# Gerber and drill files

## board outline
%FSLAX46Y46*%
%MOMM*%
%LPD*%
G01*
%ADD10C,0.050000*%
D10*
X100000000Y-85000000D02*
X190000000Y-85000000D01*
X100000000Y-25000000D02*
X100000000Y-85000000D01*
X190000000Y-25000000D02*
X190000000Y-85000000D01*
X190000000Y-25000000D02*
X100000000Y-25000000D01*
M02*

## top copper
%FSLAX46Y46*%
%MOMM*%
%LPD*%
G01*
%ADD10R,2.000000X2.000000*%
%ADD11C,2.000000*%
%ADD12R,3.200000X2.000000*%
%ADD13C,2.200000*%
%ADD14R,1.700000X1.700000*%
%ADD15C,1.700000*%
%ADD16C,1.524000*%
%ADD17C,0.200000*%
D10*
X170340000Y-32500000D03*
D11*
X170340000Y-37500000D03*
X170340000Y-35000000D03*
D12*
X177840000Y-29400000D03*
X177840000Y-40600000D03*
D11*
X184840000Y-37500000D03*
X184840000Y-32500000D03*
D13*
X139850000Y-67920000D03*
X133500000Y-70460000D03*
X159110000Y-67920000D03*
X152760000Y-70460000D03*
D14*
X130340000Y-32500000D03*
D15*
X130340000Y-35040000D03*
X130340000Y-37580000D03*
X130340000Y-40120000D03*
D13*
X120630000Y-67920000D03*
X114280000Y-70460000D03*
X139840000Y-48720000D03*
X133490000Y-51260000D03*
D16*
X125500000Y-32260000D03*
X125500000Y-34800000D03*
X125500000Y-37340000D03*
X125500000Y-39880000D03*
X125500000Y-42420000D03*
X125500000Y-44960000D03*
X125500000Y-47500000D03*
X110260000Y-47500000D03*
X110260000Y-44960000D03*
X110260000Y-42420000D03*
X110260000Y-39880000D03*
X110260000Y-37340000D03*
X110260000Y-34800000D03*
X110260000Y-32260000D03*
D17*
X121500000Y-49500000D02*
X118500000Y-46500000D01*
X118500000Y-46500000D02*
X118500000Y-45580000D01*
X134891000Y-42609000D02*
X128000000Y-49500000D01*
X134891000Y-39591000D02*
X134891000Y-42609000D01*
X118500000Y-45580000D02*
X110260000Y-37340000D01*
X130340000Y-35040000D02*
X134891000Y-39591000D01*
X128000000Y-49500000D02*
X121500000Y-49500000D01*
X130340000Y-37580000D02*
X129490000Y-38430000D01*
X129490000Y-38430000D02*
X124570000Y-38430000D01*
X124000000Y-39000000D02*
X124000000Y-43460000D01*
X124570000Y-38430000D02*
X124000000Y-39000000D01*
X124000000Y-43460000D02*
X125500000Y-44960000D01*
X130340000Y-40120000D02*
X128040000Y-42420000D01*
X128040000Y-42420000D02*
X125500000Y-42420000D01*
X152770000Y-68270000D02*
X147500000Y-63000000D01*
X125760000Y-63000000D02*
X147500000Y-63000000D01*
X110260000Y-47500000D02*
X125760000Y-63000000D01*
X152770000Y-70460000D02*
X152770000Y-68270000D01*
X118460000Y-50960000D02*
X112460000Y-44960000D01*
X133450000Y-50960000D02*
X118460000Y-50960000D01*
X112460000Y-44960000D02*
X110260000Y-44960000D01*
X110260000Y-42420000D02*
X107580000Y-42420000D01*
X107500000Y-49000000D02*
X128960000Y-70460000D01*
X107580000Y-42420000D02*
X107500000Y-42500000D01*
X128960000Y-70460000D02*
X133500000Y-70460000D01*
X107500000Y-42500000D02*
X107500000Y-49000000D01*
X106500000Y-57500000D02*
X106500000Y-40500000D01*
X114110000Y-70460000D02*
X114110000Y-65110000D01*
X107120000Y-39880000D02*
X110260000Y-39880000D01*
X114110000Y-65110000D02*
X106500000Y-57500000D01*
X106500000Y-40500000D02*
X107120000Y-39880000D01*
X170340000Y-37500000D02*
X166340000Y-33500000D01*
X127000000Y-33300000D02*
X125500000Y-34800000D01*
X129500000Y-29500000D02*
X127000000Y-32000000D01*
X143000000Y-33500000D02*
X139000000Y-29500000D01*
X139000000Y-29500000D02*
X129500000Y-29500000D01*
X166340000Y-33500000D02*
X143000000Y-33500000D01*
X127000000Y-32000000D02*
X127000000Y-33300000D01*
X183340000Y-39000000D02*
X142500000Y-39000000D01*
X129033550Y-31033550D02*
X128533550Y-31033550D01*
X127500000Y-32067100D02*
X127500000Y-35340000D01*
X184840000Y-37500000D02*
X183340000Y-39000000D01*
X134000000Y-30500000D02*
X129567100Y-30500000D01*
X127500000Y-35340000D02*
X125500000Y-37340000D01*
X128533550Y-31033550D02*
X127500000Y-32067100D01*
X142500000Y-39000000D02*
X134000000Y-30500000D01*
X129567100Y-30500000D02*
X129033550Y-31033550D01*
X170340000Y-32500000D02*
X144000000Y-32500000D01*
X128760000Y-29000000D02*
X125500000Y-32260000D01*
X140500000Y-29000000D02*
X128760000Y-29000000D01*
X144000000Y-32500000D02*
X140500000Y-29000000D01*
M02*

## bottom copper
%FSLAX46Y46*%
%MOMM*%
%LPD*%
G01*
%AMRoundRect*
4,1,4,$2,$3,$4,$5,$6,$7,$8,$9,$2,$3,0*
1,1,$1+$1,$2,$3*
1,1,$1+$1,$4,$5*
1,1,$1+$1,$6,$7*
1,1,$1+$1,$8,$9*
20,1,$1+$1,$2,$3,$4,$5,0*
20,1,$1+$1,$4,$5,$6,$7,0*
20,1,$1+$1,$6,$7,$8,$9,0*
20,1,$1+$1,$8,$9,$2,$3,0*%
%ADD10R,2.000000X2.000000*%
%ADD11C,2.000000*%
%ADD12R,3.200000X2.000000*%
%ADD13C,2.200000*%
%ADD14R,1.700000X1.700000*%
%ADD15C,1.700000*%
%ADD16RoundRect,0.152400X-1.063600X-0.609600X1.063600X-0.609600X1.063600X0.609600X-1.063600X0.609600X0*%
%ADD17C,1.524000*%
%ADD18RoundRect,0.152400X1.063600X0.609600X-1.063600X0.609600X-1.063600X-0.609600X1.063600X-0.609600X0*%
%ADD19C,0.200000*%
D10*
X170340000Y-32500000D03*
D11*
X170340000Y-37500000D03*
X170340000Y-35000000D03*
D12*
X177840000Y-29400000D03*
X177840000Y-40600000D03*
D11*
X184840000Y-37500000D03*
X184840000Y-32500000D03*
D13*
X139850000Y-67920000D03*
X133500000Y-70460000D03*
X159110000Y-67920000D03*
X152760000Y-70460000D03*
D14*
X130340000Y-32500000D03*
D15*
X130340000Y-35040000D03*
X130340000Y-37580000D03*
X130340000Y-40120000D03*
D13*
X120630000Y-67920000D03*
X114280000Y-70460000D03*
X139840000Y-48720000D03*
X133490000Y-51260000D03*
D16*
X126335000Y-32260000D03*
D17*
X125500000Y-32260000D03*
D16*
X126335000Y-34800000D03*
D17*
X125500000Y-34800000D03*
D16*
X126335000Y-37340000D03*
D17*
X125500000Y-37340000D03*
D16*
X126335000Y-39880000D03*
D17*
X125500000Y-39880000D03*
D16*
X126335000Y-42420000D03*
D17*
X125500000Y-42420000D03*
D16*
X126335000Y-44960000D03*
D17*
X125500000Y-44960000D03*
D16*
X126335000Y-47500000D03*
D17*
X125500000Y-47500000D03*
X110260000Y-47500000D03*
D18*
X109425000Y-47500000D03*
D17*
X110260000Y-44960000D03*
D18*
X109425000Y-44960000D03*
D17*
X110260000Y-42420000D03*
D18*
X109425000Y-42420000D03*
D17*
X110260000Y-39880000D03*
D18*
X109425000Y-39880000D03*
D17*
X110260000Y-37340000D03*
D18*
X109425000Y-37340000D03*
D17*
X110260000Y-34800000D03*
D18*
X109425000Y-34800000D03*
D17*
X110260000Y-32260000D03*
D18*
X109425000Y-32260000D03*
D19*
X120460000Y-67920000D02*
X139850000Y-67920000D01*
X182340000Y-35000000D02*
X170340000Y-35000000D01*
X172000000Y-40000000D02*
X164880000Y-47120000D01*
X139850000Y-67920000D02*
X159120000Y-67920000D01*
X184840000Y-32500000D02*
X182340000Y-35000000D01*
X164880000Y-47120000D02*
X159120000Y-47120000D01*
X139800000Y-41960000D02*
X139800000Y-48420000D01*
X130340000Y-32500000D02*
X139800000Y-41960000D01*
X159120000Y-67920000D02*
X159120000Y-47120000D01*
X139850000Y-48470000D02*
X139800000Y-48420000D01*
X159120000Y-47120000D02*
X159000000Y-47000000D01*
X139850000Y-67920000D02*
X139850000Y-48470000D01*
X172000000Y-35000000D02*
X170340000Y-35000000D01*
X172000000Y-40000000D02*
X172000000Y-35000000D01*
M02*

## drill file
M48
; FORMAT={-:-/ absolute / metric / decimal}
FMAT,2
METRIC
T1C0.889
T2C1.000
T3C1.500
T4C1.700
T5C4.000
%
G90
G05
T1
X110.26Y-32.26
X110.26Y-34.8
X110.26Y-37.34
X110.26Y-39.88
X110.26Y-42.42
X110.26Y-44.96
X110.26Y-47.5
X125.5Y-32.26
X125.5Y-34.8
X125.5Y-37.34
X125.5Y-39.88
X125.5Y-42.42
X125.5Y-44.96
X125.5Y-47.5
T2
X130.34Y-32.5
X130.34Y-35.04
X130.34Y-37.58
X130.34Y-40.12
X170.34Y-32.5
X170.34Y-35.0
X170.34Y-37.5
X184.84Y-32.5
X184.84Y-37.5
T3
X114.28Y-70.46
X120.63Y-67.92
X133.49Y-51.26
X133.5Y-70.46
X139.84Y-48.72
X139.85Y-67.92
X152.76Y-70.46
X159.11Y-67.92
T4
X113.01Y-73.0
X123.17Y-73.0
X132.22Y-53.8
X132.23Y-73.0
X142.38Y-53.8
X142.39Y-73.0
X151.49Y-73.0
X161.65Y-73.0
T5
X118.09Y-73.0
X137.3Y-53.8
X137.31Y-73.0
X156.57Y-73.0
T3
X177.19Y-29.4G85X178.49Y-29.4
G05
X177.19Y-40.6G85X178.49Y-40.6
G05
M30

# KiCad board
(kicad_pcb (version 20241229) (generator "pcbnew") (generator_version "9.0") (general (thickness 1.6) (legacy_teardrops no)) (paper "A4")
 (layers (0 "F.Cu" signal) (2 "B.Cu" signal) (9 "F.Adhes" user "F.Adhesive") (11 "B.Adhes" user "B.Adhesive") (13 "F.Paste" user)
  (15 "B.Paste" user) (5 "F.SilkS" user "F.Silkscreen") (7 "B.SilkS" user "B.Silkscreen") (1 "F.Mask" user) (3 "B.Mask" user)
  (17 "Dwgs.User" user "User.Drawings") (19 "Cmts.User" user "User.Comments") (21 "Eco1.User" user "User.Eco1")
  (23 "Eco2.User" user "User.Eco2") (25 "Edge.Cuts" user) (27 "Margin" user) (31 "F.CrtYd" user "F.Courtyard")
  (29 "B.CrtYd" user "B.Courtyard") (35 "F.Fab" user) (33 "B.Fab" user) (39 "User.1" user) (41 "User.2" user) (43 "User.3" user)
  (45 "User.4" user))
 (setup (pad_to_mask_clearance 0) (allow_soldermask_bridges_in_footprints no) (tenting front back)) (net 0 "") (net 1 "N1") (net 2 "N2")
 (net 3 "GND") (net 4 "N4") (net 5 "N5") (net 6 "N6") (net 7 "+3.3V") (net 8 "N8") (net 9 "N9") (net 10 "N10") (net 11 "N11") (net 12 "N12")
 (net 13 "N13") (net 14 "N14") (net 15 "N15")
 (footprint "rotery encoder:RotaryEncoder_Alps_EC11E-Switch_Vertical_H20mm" (layer "F.Cu") (at 170.34 32.5)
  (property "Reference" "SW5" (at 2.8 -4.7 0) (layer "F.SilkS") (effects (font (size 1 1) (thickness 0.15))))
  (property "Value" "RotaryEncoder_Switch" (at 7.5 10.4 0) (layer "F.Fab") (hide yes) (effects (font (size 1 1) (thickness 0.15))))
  (pad "A" thru_hole rect (at 0 0) (size 2 2) (drill 1) (layers "*.Cu" "*.Mask") (remove_unused_layers no) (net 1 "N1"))
  (pad "B" thru_hole circle (at 0 5) (size 2 2) (drill 1) (layers "*.Cu" "*.Mask") (remove_unused_layers no) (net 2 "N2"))
  (pad "C" thru_hole circle (at 0 2.5) (size 2 2) (drill 1) (layers "*.Cu" "*.Mask") (remove_unused_layers no) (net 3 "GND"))
  (pad "MP" thru_hole rect (at 7.5 -3.1) (size 3.2 2) (drill oval 2.8 1.5) (layers "*.Cu" "*.Mask") (remove_unused_layers no))
  (pad "MP" thru_hole rect (at 7.5 8.1) (size 3.2 2) (drill oval 2.8 1.5) (layers "*.Cu" "*.Mask") (remove_unused_layers no))
  (pad "S1" thru_hole circle (at 14.5 5) (size 2 2) (drill 1) (layers "*.Cu" "*.Mask") (remove_unused_layers no) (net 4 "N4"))
  (pad "S2" thru_hole circle (at 14.5 0) (size 2 2) (drill 1) (layers "*.Cu" "*.Mask") (remove_unused_layers no) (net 3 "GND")))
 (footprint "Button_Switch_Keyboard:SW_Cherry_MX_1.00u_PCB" (layer "F.Cu") (at 139.85 67.92)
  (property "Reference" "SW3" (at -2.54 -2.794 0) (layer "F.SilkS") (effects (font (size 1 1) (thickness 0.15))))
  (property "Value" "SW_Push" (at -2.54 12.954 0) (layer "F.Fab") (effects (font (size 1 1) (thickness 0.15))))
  (pad "" np_thru_hole circle (at -7.62 5.08) (size 1.7 1.7) (drill 1.7) (layers "*.Cu" "*.Mask"))
  (pad "" np_thru_hole circle (at -2.54 5.08) (size 4 4) (drill 4) (layers "*.Cu" "*.Mask"))
  (pad "" np_thru_hole circle (at 2.54 5.08) (size 1.7 1.7) (drill 1.7) (layers "*.Cu" "*.Mask"))
  (pad "1" thru_hole circle (at 0 0) (size 2.2 2.2) (drill 1.5) (layers "*.Cu" "*.Mask") (remove_unused_layers no) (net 3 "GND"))
  (pad "2" thru_hole circle (at -6.35 2.54) (size 2.2 2.2) (drill 1.5) (layers "*.Cu" "*.Mask") (remove_unused_layers no) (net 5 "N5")))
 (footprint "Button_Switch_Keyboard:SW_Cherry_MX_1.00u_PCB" (layer "F.Cu") (at 159.11 67.92)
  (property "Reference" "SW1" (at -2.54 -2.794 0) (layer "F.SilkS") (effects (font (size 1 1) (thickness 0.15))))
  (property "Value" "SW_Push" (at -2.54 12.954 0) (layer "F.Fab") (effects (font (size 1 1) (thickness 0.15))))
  (pad "" np_thru_hole circle (at -7.62 5.08) (size 1.7 1.7) (drill 1.7) (layers "*.Cu" "*.Mask"))
  (pad "" np_thru_hole circle (at -2.54 5.08) (size 4 4) (drill 4) (layers "*.Cu" "*.Mask"))
  (pad "" np_thru_hole circle (at 2.54 5.08) (size 1.7 1.7) (drill 1.7) (layers "*.Cu" "*.Mask"))
  (pad "1" thru_hole circle (at 0 0) (size 2.2 2.2) (drill 1.5) (layers "*.Cu" "*.Mask") (remove_unused_layers no) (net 3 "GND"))
  (pad "2" thru_hole circle (at -6.35 2.54) (size 2.2 2.2) (drill 1.5) (layers "*.Cu" "*.Mask") (remove_unused_layers no) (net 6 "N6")))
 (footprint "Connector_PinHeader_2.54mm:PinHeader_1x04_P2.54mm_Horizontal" (layer "F.Cu") (at 130.34 32.5)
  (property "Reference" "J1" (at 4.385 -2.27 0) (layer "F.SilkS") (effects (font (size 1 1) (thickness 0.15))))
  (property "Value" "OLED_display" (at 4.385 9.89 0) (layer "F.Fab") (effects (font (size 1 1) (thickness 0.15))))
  (pad "1" thru_hole rect (at 0 0) (size 1.7 1.7) (drill 1) (layers "*.Cu" "*.Mask") (remove_unused_layers no) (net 3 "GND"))
  (pad "2" thru_hole circle (at 0 2.54) (size 1.7 1.7) (drill 1) (layers "*.Cu" "*.Mask") (remove_unused_layers no) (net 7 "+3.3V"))
  (pad "3" thru_hole circle (at 0 5.08) (size 1.7 1.7) (drill 1) (layers "*.Cu" "*.Mask") (remove_unused_layers no) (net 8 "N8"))
  (pad "4" thru_hole circle (at 0 7.62) (size 1.7 1.7) (drill 1) (layers "*.Cu" "*.Mask") (remove_unused_layers no) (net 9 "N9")))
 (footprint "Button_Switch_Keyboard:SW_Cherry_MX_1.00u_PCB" (layer "F.Cu") (at 120.63 67.92)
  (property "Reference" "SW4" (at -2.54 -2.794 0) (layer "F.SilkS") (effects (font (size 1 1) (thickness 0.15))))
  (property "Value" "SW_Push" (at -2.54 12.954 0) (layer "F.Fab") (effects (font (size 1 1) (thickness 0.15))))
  (pad "" np_thru_hole circle (at -7.62 5.08) (size 1.7 1.7) (drill 1.7) (layers "*.Cu" "*.Mask"))
  (pad "" np_thru_hole circle (at -2.54 5.08) (size 4 4) (drill 4) (layers "*.Cu" "*.Mask"))
  (pad "" np_thru_hole circle (at 2.54 5.08) (size 1.7 1.7) (drill 1.7) (layers "*.Cu" "*.Mask"))
  (pad "1" thru_hole circle (at 0 0) (size 2.2 2.2) (drill 1.5) (layers "*.Cu" "*.Mask") (remove_unused_layers no) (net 3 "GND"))
  (pad "2" thru_hole circle (at -6.35 2.54) (size 2.2 2.2) (drill 1.5) (layers "*.Cu" "*.Mask") (remove_unused_layers no) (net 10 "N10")))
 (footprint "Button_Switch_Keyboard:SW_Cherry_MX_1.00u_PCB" (layer "F.Cu") (at 139.84 48.72)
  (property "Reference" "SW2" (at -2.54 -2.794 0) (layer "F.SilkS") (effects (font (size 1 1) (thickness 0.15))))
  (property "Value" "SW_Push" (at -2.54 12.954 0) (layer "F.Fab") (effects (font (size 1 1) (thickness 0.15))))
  (pad "" np_thru_hole circle (at -7.62 5.08) (size 1.7 1.7) (drill 1.7) (layers "*.Cu" "*.Mask"))
  (pad "" np_thru_hole circle (at -2.54 5.08) (size 4 4) (drill 4) (layers "*.Cu" "*.Mask"))
  (pad "" np_thru_hole circle (at 2.54 5.08) (size 1.7 1.7) (drill 1.7) (layers "*.Cu" "*.Mask"))
  (pad "1" thru_hole circle (at 0 0) (size 2.2 2.2) (drill 1.5) (layers "*.Cu" "*.Mask") (remove_unused_layers no) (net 3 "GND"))
  (pad "2" thru_hole circle (at -6.35 2.54) (size 2.2 2.2) (drill 1.5) (layers "*.Cu" "*.Mask") (remove_unused_layers no) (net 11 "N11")))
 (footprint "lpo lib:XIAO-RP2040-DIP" (layer "B.Cu") (at 117.88 39.88 180)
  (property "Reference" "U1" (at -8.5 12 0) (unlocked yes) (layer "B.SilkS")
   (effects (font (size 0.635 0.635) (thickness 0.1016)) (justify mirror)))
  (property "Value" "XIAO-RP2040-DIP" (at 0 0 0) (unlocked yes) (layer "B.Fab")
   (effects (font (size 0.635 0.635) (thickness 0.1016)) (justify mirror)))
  (pad "1" smd roundrect (at -8.455 7.62) (size 2.432 1.524) (layers "B.Cu" "B.Mask") (roundrect_rratio 0.1) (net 1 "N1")
   (thermal_bridge_angle 45))
  (pad "1" thru_hole circle (at -7.62 7.62) (size 1.524 1.524) (drill 0.889) (layers "*.Cu" "*.Mask") (remove_unused_layers no) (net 1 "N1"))
  (pad "2" smd roundrect (at -8.455 5.08) (size 2.432 1.524) (layers "B.Cu" "B.Mask") (roundrect_rratio 0.1) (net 2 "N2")
   (thermal_bridge_angle 45))
  (pad "2" thru_hole circle (at -7.62 5.08) (size 1.524 1.524) (drill 0.889) (layers "*.Cu" "*.Mask") (remove_unused_layers no) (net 2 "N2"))
  (pad "3" smd roundrect (at -8.455 2.54) (size 2.432 1.524) (layers "B.Cu" "B.Mask") (roundrect_rratio 0.1) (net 4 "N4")
   (thermal_bridge_angle 45))
  (pad "3" thru_hole circle (at -7.62 2.54) (size 1.524 1.524) (drill 0.889) (layers "*.Cu" "*.Mask") (remove_unused_layers no) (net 4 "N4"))
  (pad "4" smd roundrect (at -8.455 0) (size 2.432 1.524) (layers "B.Cu" "B.Mask") (roundrect_rratio 0.1) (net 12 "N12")
   (thermal_bridge_angle 45))
  (pad "4" thru_hole circle (at -7.62 0) (size 1.524 1.524) (drill 0.889) (layers "*.Cu" "*.Mask") (remove_unused_layers no) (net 12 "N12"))
  (pad "5" smd roundrect (at -8.455 -2.54) (size 2.432 1.524) (layers "B.Cu" "B.Mask") (roundrect_rratio 0.1) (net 9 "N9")
   (thermal_bridge_angle 45))
  (pad "5" thru_hole circle (at -7.62 -2.54) (size 1.524 1.524) (drill 0.889) (layers "*.Cu" "*.Mask") (remove_unused_layers no)
   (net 9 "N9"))
  (pad "6" smd roundrect (at -8.455 -5.08) (size 2.432 1.524) (layers "B.Cu" "B.Mask") (roundrect_rratio 0.1) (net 8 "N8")
   (thermal_bridge_angle 45))
  (pad "6" thru_hole circle (at -7.62 -5.08) (size 1.524 1.524) (drill 0.889) (layers "*.Cu" "*.Mask") (remove_unused_layers no)
   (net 8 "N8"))
  (pad "7" smd roundrect (at -8.455 -7.62) (size 2.432 1.524) (layers "B.Cu" "B.Mask") (roundrect_rratio 0.1) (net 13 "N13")
   (thermal_bridge_angle 45))
  (pad "7" thru_hole circle (at -7.62 -7.62) (size 1.524 1.524) (drill 0.889) (layers "*.Cu" "*.Mask") (remove_unused_layers no)
   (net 13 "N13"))
  (pad "8" thru_hole circle (at 7.62 -7.62 180) (size 1.524 1.524) (drill 0.889) (layers "*.Cu" "*.Mask") (remove_unused_layers no)
   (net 6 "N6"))
  (pad "8" smd roundrect (at 8.455 -7.62 180) (size 2.432 1.524) (layers "B.Cu" "B.Mask") (roundrect_rratio 0.1) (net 6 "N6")
   (thermal_bridge_angle 45))
  (pad "9" thru_hole circle (at 7.62 -5.08 180) (size 1.524 1.524) (drill 0.889) (layers "*.Cu" "*.Mask") (remove_unused_layers no)
   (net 11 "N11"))
  (pad "9" smd roundrect (at 8.455 -5.08 180) (size 2.432 1.524) (layers "B.Cu" "B.Mask") (roundrect_rratio 0.1) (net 11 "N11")
   (thermal_bridge_angle 45))
  (pad "10" thru_hole circle (at 7.62 -2.54 180) (size 1.524 1.524) (drill 0.889) (layers "*.Cu" "*.Mask") (remove_unused_layers no)
   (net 5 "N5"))
  (pad "10" smd roundrect (at 8.455 -2.54 180) (size 2.432 1.524) (layers "B.Cu" "B.Mask") (roundrect_rratio 0.1) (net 5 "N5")
   (thermal_bridge_angle 45))
  (pad "11" thru_hole circle (at 7.62 0 180) (size 1.524 1.524) (drill 0.889) (layers "*.Cu" "*.Mask") (remove_unused_layers no)
   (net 10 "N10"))
  (pad "11" smd roundrect (at 8.455 0 180) (size 2.432 1.524) (layers "B.Cu" "B.Mask") (roundrect_rratio 0.1) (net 10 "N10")
   (thermal_bridge_angle 45))
  (pad "12" thru_hole circle (at 7.62 2.54 180) (size 1.524 1.524) (drill 0.889) (layers "*.Cu" "*.Mask") (remove_unused_layers no)
   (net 7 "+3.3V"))
  (pad "12" smd roundrect (at 8.455 2.54 180) (size 2.432 1.524) (layers "B.Cu" "B.Mask") (roundrect_rratio 0.1) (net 7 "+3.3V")
   (thermal_bridge_angle 45))
  (pad "13" thru_hole circle (at 7.62 5.08 180) (size 1.524 1.524) (drill 0.889) (layers "*.Cu" "*.Mask") (remove_unused_layers no)
   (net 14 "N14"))
  (pad "13" smd roundrect (at 8.455 5.08 180) (size 2.432 1.524) (layers "B.Cu" "B.Mask") (roundrect_rratio 0.1) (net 14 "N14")
   (thermal_bridge_angle 45))
  (pad "14" thru_hole circle (at 7.62 7.62 180) (size 1.524 1.524) (drill 0.889) (layers "*.Cu" "*.Mask") (remove_unused_layers no)
   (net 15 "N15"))
  (pad "14" smd roundrect (at 8.455 7.62 180) (size 2.432 1.524) (layers "B.Cu" "B.Mask") (roundrect_rratio 0.1) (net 15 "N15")
   (thermal_bridge_angle 45)))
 (gr_line (start 100 85) (end 190 85) (stroke (width 0.05) (type default)) (layer "Edge.Cuts"))
 (gr_line (start 100 25) (end 100 85) (stroke (width 0.05) (type default)) (layer "Edge.Cuts"))
 (gr_line (start 190 25) (end 190 85) (stroke (width 0.05) (type default)) (layer "Edge.Cuts"))
 (gr_line (start 190 25) (end 100 25) (stroke (width 0.05) (type default)) (layer "Edge.Cuts"))
 (segment (start 121.5 49.5) (end 118.5 46.5) (width 0.2) (layer "F.Cu") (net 7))
 (segment (start 118.5 46.5) (end 118.5 45.58) (width 0.2) (layer "F.Cu") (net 7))
 (segment (start 134.891 42.609) (end 128 49.5) (width 0.2) (layer "F.Cu") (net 7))
 (segment (start 134.891 39.591) (end 134.891 42.609) (width 0.2) (layer "F.Cu") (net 7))
 (segment (start 118.5 45.58) (end 110.26 37.34) (width 0.2) (layer "F.Cu") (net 7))
 (segment (start 130.34 35.04) (end 134.891 39.591) (width 0.2) (layer "F.Cu") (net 7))
 (segment (start 128 49.5) (end 121.5 49.5) (width 0.2) (layer "F.Cu") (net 7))
 (segment (start 120.46 67.92) (end 139.85 67.92) (width 0.2) (layer "B.Cu") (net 3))
 (segment (start 182.34 35) (end 170.34 35) (width 0.2) (layer "B.Cu") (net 3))
 (segment (start 172 40) (end 164.88 47.12) (width 0.2) (layer "B.Cu") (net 3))
 (segment (start 139.85 67.92) (end 159.12 67.92) (width 0.2) (layer "B.Cu") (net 3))
 (segment (start 184.84 32.5) (end 182.34 35) (width 0.2) (layer "B.Cu") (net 3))
 (segment (start 164.88 47.12) (end 159.12 47.12) (width 0.2) (layer "B.Cu") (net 3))
 (segment (start 139.8 41.96) (end 139.8 48.42) (width 0.2) (layer "B.Cu") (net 3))
 (segment (start 130.34 32.5) (end 139.8 41.96) (width 0.2) (layer "B.Cu") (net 3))
 (segment (start 159.12 67.92) (end 159.12 47.12) (width 0.2) (layer "B.Cu") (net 3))
 (segment (start 139.85 48.47) (end 139.8 48.42) (width 0.2) (layer "B.Cu") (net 3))
 (segment (start 159.12 47.12) (end 159 47) (width 0.2) (layer "B.Cu") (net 3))
 (segment (start 139.85 67.92) (end 139.85 48.47) (width 0.2) (layer "B.Cu") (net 3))
 (segment (start 172 35) (end 170.34 35) (width 0.2) (layer "B.Cu") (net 3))
 (segment (start 172 40) (end 172 35) (width 0.2) (layer "B.Cu") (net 3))
 (segment (start 130.34 37.58) (end 129.49 38.43) (width 0.2) (layer "F.Cu") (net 8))
 (segment (start 129.49 38.43) (end 124.57 38.43) (width 0.2) (layer "F.Cu") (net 8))
 (segment (start 124 39) (end 124 43.46) (width 0.2) (layer "F.Cu") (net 8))
 (segment (start 124.57 38.43) (end 124 39) (width 0.2) (layer "F.Cu") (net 8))
 (segment (start 124 43.46) (end 125.5 44.96) (width 0.2) (layer "F.Cu") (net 8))
 (segment (start 130.34 40.12) (end 128.04 42.42) (width 0.2) (layer "F.Cu") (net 9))
 (segment (start 128.04 42.42) (end 125.5 42.42) (width 0.2) (layer "F.Cu") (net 9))
 (segment (start 152.77 68.27) (end 147.5 63) (width 0.2) (layer "F.Cu") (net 6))
 (segment (start 125.76 63) (end 147.5 63) (width 0.2) (layer "F.Cu") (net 6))
 (segment (start 110.26 47.5) (end 125.76 63) (width 0.2) (layer "F.Cu") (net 6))
 (segment (start 152.77 70.46) (end 152.77 68.27) (width 0.2) (layer "F.Cu") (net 6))
 (segment (start 118.46 50.96) (end 112.46 44.96) (width 0.2) (layer "F.Cu") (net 11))
 (segment (start 133.45 50.96) (end 118.46 50.96) (width 0.2) (layer "F.Cu") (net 11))
 (segment (start 112.46 44.96) (end 110.26 44.96) (width 0.2) (layer "F.Cu") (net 11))
 (segment (start 110.26 42.42) (end 107.58 42.42) (width 0.2) (layer "F.Cu") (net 5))
 (segment (start 107.5 49) (end 128.96 70.46) (width 0.2) (layer "F.Cu") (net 5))
 (segment (start 107.58 42.42) (end 107.5 42.5) (width 0.2) (layer "F.Cu") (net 5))
 (segment (start 128.96 70.46) (end 133.5 70.46) (width 0.2) (layer "F.Cu") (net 5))
 (segment (start 107.5 42.5) (end 107.5 49) (width 0.2) (layer "F.Cu") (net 5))
 (segment (start 106.5 57.5) (end 106.5 40.5) (width 0.2) (layer "F.Cu") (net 10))
 (segment (start 114.11 70.46) (end 114.11 65.11) (width 0.2) (layer "F.Cu") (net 10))
 (segment (start 107.12 39.88) (end 110.26 39.88) (width 0.2) (layer "F.Cu") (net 10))
 (segment (start 114.11 65.11) (end 106.5 57.5) (width 0.2) (layer "F.Cu") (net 10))
 (segment (start 106.5 40.5) (end 107.12 39.88) (width 0.2) (layer "F.Cu") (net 10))
 (segment (start 170.34 37.5) (end 166.34 33.5) (width 0.2) (layer "F.Cu") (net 2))
 (segment (start 127 33.3) (end 125.5 34.8) (width 0.2) (layer "F.Cu") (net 2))
 (segment (start 129.5 29.5) (end 127 32) (width 0.2) (layer "F.Cu") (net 2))
 (segment (start 143 33.5) (end 139 29.5) (width 0.2) (layer "F.Cu") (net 2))
 (segment (start 139 29.5) (end 129.5 29.5) (width 0.2) (layer "F.Cu") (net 2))
 (segment (start 166.34 33.5) (end 143 33.5) (width 0.2) (layer "F.Cu") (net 2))
 (segment (start 127 32) (end 127 33.3) (width 0.2) (layer "F.Cu") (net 2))
 (segment (start 183.34 39) (end 142.5 39) (width 0.2) (layer "F.Cu") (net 4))
 (segment (start 129.03355 31.03355) (end 128.53355 31.03355) (width 0.2) (layer "F.Cu") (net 4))
 (segment (start 127.5 32.0671) (end 127.5 35.34) (width 0.2) (layer "F.Cu") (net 4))
 (segment (start 184.84 37.5) (end 183.34 39) (width 0.2) (layer "F.Cu") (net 4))
 (segment (start 134 30.5) (end 129.5671 30.5) (width 0.2) (layer "F.Cu") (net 4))
 (segment (start 127.5 35.34) (end 125.5 37.34) (width 0.2) (layer "F.Cu") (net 4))
 (segment (start 128.53355 31.03355) (end 127.5 32.0671) (width 0.2) (layer "F.Cu") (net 4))
 (segment (start 142.5 39) (end 134 30.5) (width 0.2) (layer "F.Cu") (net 4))
 (segment (start 129.5671 30.5) (end 129.03355 31.03355) (width 0.2) (layer "F.Cu") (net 4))
 (segment (start 170.34 32.5) (end 144 32.5) (width 0.2) (layer "F.Cu") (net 1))
 (segment (start 128.76 29) (end 125.5 32.26) (width 0.2) (layer "F.Cu") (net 1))
 (segment (start 140.5 29) (end 128.76 29) (width 0.2) (layer "F.Cu") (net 1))
 (segment (start 144 32.5) (end 140.5 29) (width 0.2) (layer "F.Cu") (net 1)))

